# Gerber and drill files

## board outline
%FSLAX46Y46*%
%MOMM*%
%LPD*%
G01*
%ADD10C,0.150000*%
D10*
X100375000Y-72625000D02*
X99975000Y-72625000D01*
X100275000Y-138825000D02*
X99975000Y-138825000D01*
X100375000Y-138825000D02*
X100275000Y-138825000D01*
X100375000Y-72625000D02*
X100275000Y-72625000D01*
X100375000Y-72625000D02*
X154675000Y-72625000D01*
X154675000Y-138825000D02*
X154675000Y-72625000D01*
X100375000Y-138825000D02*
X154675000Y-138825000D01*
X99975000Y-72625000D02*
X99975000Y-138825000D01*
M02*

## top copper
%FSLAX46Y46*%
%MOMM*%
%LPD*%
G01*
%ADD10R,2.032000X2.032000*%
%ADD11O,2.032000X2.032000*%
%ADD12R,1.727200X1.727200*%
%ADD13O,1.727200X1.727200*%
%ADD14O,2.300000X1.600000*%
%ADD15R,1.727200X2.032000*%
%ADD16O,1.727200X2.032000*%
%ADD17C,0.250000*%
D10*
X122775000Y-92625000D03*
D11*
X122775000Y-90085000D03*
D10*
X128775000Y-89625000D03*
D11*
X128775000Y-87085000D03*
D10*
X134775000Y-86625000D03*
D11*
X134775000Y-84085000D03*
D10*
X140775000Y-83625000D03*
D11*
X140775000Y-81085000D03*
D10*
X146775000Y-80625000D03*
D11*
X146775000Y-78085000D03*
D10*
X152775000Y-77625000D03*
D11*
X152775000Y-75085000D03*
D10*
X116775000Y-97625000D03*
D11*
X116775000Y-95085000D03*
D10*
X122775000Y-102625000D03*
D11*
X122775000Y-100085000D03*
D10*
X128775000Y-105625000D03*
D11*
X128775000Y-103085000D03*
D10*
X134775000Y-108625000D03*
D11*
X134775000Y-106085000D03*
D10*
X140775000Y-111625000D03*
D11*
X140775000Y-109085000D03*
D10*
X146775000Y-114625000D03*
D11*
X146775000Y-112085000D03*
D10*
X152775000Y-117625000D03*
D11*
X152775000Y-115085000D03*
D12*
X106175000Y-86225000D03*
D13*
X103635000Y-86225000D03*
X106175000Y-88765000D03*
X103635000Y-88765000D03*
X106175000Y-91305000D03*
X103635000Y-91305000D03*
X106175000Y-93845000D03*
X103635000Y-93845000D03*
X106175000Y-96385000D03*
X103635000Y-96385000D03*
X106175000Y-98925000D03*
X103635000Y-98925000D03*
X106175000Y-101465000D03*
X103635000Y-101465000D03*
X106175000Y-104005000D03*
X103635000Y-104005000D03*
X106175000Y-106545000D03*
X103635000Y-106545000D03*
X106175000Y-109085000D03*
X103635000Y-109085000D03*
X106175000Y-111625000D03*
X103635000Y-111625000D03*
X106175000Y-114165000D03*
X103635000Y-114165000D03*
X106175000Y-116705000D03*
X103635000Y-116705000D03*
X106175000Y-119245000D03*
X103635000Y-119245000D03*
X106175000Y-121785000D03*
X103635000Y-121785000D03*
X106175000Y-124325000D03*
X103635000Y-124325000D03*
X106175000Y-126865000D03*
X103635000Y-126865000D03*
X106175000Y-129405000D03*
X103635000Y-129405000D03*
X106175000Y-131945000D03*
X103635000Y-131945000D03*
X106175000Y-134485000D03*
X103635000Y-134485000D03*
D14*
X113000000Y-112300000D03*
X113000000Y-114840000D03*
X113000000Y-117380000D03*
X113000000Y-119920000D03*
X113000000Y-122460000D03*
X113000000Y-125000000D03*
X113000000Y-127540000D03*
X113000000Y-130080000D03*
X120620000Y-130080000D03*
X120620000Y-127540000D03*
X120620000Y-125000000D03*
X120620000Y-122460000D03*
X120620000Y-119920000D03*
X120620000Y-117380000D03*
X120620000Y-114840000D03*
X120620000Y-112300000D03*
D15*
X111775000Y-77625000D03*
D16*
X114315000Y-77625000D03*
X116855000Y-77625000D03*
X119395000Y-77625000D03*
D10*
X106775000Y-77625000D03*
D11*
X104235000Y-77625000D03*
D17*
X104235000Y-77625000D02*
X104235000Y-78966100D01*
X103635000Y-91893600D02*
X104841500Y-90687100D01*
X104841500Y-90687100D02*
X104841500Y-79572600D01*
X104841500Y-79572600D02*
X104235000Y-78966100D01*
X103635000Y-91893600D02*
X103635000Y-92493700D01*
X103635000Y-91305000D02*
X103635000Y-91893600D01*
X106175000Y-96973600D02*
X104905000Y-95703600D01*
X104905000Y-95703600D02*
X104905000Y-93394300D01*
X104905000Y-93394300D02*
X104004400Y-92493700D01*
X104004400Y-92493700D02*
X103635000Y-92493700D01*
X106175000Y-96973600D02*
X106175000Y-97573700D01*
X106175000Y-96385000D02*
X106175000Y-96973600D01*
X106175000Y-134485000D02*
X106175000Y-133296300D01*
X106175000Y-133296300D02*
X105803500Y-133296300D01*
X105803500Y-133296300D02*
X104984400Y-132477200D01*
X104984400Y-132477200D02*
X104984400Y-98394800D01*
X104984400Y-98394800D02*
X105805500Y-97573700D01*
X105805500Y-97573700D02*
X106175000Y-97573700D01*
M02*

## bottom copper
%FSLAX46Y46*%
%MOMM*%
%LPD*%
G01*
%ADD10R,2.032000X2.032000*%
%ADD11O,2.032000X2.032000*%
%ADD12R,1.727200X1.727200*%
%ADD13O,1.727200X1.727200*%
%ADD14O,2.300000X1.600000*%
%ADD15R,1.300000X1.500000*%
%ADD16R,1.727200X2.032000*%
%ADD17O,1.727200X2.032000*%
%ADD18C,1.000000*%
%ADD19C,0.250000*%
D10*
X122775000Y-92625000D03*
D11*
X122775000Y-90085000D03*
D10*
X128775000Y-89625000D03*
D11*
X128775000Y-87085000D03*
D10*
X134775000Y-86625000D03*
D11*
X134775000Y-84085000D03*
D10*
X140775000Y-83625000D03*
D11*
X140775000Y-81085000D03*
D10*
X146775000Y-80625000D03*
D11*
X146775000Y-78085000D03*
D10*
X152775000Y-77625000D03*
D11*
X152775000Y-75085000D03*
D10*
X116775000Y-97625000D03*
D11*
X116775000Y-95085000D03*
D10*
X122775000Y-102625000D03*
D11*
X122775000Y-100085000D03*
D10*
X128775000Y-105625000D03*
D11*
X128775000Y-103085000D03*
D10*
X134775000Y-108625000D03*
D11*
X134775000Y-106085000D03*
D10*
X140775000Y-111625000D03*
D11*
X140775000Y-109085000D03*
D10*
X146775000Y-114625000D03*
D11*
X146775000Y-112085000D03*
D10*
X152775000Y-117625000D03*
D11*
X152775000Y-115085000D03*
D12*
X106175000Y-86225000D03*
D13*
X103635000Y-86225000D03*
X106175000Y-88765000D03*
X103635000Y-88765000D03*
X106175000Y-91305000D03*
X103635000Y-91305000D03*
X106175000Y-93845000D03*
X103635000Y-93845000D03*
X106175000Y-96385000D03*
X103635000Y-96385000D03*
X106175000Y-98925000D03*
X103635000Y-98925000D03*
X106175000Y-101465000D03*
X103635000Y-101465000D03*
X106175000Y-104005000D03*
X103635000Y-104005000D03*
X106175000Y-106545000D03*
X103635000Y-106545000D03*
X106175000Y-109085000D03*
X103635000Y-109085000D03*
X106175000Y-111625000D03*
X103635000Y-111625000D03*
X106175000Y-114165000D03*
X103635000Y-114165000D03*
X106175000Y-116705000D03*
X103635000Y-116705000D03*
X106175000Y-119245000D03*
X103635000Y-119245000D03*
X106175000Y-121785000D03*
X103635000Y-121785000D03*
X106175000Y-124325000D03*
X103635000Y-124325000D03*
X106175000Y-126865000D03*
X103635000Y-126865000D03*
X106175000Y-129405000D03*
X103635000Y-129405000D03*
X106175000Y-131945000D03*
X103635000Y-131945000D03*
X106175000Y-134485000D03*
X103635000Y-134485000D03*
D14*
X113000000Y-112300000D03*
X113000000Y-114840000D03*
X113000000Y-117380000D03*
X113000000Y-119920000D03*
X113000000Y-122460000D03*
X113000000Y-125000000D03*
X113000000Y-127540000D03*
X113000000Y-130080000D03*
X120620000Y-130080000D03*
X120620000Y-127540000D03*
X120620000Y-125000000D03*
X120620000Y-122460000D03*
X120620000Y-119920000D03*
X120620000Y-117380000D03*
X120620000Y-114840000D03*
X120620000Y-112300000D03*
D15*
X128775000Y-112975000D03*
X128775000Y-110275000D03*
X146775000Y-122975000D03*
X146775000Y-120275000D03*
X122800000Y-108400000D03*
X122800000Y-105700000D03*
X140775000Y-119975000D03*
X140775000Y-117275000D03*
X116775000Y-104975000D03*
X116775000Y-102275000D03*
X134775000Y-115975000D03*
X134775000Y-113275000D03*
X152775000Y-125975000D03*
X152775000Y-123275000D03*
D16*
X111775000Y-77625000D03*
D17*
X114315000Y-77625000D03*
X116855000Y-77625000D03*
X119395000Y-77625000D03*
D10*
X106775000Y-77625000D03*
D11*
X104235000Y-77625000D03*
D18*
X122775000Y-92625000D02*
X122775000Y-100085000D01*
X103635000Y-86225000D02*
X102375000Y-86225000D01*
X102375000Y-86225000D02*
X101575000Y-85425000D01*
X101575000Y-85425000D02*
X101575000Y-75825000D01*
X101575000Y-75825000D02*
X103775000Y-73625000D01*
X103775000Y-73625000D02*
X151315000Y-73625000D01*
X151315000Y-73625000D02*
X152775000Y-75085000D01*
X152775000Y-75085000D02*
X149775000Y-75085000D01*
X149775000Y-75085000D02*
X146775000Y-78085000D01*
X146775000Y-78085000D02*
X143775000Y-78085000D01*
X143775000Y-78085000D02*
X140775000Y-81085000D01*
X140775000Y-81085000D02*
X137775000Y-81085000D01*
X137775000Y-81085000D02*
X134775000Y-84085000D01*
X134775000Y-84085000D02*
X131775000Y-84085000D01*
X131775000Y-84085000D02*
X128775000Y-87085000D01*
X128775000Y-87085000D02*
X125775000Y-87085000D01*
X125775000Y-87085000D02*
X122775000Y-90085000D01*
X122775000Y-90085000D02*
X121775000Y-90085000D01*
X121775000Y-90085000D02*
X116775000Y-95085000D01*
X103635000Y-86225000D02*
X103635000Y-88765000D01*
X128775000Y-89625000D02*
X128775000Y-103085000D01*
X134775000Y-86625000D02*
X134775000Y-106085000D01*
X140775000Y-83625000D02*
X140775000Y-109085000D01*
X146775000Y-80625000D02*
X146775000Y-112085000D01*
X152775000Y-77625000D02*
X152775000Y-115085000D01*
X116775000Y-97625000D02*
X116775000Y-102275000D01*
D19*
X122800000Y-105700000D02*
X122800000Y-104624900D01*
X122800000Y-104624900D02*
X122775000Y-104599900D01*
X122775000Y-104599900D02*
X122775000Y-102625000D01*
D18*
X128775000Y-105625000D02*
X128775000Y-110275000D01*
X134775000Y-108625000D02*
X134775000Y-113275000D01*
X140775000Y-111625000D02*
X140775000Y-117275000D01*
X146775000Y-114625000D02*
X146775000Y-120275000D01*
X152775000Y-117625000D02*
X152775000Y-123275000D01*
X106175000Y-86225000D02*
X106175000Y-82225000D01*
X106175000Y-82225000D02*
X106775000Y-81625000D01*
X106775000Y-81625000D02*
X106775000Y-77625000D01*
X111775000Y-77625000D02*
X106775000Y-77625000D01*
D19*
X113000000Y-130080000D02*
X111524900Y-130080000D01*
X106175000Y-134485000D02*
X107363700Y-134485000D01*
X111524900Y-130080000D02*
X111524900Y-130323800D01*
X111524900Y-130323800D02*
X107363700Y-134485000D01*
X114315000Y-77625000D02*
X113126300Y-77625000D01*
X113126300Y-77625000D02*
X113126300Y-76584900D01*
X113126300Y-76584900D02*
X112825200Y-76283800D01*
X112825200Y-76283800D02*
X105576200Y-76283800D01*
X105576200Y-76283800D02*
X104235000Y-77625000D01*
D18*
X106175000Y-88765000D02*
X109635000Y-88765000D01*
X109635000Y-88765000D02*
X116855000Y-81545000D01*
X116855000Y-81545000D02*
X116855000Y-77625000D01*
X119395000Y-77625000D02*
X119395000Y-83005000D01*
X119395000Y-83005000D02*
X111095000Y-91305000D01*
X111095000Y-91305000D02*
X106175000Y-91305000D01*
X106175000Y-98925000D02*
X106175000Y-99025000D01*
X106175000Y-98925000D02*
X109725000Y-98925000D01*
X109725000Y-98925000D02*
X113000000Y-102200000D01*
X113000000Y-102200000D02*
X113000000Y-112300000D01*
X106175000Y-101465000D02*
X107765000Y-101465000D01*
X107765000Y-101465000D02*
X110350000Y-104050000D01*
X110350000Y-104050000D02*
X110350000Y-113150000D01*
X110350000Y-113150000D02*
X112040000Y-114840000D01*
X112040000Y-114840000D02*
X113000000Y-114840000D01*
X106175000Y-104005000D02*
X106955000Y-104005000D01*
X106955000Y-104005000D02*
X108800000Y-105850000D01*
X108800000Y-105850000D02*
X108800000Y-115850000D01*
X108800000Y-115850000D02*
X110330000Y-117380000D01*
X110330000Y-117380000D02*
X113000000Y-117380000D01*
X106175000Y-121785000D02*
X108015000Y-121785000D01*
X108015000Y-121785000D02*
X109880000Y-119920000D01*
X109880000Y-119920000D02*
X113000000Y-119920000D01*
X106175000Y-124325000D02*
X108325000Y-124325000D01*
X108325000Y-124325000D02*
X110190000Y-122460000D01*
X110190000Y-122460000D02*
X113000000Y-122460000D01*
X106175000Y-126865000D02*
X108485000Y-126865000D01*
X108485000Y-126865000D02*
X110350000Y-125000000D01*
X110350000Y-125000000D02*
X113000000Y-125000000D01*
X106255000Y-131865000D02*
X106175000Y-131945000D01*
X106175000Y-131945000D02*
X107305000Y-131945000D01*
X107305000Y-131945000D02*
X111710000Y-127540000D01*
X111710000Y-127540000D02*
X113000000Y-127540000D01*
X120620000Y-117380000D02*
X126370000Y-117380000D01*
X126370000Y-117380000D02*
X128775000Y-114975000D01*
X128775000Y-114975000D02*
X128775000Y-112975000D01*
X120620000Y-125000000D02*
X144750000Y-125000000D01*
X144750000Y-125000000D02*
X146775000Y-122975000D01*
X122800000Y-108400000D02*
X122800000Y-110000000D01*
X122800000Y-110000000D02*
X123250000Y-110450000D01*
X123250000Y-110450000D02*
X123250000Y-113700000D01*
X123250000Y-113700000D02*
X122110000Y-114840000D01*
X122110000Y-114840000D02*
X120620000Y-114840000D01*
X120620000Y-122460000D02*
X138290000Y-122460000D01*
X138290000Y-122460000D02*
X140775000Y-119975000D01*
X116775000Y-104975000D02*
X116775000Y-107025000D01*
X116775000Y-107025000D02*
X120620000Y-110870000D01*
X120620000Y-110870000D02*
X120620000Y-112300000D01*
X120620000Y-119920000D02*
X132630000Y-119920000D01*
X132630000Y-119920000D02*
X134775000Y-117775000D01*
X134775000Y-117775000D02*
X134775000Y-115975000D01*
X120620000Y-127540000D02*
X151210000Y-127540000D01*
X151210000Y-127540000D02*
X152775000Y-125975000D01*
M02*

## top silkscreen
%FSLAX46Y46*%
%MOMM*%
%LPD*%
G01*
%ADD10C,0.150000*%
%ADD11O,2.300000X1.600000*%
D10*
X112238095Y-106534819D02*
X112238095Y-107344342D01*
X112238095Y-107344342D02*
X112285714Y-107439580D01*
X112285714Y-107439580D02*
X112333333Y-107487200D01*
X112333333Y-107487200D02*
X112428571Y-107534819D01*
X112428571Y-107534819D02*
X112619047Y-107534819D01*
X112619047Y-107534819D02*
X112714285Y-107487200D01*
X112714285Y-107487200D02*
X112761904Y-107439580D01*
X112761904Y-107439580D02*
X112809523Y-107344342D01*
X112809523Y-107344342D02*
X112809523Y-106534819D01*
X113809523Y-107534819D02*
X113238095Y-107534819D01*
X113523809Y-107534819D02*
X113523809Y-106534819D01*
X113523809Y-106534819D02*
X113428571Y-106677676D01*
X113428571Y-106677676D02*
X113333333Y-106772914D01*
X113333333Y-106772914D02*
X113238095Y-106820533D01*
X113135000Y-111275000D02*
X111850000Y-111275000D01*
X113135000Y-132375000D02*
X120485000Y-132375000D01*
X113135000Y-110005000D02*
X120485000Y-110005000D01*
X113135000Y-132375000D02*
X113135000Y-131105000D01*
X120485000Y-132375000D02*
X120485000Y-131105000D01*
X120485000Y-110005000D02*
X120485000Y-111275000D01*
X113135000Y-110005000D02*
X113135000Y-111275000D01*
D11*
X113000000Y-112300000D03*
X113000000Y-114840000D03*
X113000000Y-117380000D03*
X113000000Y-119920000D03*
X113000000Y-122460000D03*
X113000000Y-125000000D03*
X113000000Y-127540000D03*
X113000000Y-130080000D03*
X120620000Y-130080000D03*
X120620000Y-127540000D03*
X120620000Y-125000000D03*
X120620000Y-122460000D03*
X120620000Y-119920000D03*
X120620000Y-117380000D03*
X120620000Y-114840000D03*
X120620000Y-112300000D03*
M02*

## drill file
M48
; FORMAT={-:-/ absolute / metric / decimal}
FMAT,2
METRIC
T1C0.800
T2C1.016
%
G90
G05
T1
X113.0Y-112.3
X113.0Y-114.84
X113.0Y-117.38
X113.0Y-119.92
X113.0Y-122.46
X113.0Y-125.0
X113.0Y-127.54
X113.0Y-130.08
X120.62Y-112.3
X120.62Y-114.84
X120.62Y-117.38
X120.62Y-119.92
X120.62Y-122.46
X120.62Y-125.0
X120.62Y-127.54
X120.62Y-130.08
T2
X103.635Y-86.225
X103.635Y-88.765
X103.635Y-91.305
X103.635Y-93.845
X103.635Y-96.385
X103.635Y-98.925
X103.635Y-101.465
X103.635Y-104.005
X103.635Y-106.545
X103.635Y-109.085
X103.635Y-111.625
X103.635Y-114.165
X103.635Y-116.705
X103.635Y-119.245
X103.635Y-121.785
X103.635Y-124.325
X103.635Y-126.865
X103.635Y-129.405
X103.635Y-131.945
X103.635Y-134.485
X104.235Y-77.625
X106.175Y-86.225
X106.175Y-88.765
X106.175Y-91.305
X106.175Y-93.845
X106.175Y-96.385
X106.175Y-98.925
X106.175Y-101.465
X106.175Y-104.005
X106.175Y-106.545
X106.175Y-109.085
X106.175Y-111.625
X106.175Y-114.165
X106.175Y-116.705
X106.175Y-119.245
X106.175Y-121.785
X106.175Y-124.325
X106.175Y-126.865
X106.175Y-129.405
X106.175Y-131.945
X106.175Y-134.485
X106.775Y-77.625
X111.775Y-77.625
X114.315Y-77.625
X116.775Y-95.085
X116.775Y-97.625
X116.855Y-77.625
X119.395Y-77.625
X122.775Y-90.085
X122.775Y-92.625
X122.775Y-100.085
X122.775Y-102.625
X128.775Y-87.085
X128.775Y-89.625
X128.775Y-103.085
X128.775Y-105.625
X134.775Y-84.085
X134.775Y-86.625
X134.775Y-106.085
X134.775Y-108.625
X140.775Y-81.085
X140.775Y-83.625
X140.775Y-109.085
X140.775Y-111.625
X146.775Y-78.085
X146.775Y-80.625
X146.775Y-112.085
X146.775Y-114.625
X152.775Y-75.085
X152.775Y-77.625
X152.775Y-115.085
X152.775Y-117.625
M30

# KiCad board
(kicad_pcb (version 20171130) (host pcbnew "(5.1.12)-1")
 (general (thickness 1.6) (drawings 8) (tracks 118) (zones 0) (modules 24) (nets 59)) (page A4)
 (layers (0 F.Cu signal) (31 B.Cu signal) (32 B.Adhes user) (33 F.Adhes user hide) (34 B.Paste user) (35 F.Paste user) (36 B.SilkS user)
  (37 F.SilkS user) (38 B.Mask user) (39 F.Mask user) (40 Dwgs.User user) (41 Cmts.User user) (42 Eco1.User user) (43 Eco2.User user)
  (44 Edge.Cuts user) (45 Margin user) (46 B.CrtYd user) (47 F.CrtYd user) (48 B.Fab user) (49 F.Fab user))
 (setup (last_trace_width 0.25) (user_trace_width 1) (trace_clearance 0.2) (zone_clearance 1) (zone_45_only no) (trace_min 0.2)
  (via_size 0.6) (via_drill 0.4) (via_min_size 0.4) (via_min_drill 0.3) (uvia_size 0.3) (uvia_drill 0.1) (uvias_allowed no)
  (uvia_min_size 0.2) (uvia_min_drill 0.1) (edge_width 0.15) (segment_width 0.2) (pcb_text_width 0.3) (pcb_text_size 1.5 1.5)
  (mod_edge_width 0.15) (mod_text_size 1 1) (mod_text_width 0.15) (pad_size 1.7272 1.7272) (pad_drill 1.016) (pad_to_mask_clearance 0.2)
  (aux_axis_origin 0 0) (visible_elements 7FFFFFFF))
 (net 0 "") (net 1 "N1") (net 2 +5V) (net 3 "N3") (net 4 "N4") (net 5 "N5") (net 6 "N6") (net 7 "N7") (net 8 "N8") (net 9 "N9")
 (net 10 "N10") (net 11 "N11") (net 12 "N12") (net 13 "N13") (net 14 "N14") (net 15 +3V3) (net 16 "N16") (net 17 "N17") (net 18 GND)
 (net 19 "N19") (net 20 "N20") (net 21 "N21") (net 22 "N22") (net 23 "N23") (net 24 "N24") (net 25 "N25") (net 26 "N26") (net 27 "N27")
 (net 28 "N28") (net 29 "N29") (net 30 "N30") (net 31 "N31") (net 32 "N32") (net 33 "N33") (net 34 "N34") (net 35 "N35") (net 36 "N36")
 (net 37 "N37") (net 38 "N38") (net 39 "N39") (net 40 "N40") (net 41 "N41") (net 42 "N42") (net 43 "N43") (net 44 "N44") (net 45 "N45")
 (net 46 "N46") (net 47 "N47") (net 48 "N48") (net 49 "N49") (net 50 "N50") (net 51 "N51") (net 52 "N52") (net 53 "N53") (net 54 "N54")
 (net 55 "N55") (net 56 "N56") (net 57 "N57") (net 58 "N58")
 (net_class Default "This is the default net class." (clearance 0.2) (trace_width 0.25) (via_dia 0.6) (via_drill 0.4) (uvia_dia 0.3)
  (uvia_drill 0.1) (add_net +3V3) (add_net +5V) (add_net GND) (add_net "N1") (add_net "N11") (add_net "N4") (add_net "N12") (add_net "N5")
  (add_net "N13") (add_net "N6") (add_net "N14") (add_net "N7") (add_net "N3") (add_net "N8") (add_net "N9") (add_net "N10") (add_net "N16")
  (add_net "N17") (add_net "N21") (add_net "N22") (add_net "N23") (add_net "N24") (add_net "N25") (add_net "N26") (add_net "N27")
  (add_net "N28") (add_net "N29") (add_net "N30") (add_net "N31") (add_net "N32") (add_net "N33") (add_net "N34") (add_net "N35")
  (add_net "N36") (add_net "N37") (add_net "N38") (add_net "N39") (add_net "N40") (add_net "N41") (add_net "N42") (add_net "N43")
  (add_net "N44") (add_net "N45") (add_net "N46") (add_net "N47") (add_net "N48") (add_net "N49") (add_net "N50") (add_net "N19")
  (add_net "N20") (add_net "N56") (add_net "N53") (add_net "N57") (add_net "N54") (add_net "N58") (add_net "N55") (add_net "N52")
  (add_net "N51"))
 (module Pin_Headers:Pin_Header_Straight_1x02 (layer B.Cu) (at 122.775 92.625)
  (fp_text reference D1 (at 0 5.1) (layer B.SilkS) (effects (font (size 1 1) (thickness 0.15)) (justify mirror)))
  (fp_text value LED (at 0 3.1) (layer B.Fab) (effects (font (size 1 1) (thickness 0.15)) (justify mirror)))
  (pad 1 thru_hole rect (at 0 0) (size 2.032 2.032) (drill 1.016) (layers *.Cu *.Mask B.SilkS) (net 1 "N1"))
  (pad 2 thru_hole oval (at 0 -2.54) (size 2.032 2.032) (drill 1.016) (layers *.Cu *.Mask B.SilkS) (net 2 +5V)))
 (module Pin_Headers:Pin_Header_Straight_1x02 (layer B.Cu) (at 128.775 89.625)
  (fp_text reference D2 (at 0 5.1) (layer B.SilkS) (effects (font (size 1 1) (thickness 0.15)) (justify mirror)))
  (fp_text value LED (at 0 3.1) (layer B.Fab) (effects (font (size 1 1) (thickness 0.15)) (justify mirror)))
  (pad 1 thru_hole rect (at 0 0) (size 2.032 2.032) (drill 1.016) (layers *.Cu *.Mask B.SilkS) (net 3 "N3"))
  (pad 2 thru_hole oval (at 0 -2.54) (size 2.032 2.032) (drill 1.016) (layers *.Cu *.Mask B.SilkS) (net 2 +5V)))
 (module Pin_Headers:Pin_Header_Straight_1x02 (layer B.Cu) (at 134.775 86.625)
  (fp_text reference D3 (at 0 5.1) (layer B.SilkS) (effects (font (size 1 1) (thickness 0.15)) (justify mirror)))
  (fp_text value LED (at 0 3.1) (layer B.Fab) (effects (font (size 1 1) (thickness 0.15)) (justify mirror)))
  (pad 1 thru_hole rect (at 0 0) (size 2.032 2.032) (drill 1.016) (layers *.Cu *.Mask B.SilkS) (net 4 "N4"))
  (pad 2 thru_hole oval (at 0 -2.54) (size 2.032 2.032) (drill 1.016) (layers *.Cu *.Mask B.SilkS) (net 2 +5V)))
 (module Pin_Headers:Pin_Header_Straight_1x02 (layer B.Cu) (at 140.775 83.625)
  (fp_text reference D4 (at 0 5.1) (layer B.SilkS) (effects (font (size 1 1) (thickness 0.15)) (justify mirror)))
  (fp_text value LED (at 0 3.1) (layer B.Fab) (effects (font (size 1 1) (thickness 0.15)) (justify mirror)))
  (pad 1 thru_hole rect (at 0 0) (size 2.032 2.032) (drill 1.016) (layers *.Cu *.Mask B.SilkS) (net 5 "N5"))
  (pad 2 thru_hole oval (at 0 -2.54) (size 2.032 2.032) (drill 1.016) (layers *.Cu *.Mask B.SilkS) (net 2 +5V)))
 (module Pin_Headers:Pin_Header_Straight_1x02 (layer B.Cu) (at 146.775 80.625)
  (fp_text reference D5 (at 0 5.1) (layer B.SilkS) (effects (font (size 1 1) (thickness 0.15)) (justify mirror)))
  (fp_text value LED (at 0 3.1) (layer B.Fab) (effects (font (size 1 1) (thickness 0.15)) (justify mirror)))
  (pad 1 thru_hole rect (at 0 0) (size 2.032 2.032) (drill 1.016) (layers *.Cu *.Mask B.SilkS) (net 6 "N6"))
  (pad 2 thru_hole oval (at 0 -2.54) (size 2.032 2.032) (drill 1.016) (layers *.Cu *.Mask B.SilkS) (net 2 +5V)))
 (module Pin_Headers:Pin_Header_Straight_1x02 (layer B.Cu) (at 152.775 77.625)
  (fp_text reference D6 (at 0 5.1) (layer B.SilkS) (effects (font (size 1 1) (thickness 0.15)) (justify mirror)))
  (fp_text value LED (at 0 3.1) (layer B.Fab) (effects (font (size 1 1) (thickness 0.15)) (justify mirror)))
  (pad 1 thru_hole rect (at 0 0) (size 2.032 2.032) (drill 1.016) (layers *.Cu *.Mask B.SilkS) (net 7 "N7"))
  (pad 2 thru_hole oval (at 0 -2.54) (size 2.032 2.032) (drill 1.016) (layers *.Cu *.Mask B.SilkS) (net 2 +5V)))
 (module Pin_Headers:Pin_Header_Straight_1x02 (layer B.Cu) (at 116.775 97.625)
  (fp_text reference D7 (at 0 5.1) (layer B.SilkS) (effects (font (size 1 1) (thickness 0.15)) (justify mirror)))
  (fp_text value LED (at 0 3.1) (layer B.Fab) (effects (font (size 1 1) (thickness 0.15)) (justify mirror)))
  (pad 1 thru_hole rect (at 0 0) (size 2.032 2.032) (drill 1.016) (layers *.Cu *.Mask B.SilkS) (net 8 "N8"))
  (pad 2 thru_hole oval (at 0 -2.54) (size 2.032 2.032) (drill 1.016) (layers *.Cu *.Mask B.SilkS) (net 2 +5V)))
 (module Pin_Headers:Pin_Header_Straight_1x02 (layer B.Cu) (at 122.775 102.625)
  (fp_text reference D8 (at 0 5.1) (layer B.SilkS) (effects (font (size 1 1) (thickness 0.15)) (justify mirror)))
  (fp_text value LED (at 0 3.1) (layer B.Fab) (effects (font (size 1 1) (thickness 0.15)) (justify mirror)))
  (pad 1 thru_hole rect (at 0 0) (size 2.032 2.032) (drill 1.016) (layers *.Cu *.Mask B.SilkS) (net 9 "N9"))
  (pad 2 thru_hole oval (at 0 -2.54) (size 2.032 2.032) (drill 1.016) (layers *.Cu *.Mask B.SilkS) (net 1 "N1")))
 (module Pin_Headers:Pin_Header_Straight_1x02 (layer B.Cu) (at 128.775 105.625)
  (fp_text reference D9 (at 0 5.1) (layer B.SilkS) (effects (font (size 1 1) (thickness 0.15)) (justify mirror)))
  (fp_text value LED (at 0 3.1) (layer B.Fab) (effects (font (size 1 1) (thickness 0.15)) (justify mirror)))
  (pad 1 thru_hole rect (at 0 0) (size 2.032 2.032) (drill 1.016) (layers *.Cu *.Mask B.SilkS) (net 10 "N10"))
  (pad 2 thru_hole oval (at 0 -2.54) (size 2.032 2.032) (drill 1.016) (layers *.Cu *.Mask B.SilkS) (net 3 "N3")))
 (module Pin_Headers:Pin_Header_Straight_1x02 (layer B.Cu) (at 134.775 108.625)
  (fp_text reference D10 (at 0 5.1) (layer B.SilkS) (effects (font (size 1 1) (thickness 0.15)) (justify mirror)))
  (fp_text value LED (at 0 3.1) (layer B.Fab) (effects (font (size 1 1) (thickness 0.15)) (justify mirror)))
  (pad 1 thru_hole rect (at 0 0) (size 2.032 2.032) (drill 1.016) (layers *.Cu *.Mask B.SilkS) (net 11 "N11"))
  (pad 2 thru_hole oval (at 0 -2.54) (size 2.032 2.032) (drill 1.016) (layers *.Cu *.Mask B.SilkS) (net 4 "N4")))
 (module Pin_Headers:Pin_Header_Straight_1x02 (layer B.Cu) (at 140.775 111.625)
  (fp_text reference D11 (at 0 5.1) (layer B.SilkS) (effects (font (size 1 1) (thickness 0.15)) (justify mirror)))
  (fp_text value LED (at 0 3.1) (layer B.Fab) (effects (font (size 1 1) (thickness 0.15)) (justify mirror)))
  (pad 1 thru_hole rect (at 0 0) (size 2.032 2.032) (drill 1.016) (layers *.Cu *.Mask B.SilkS) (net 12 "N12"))
  (pad 2 thru_hole oval (at 0 -2.54) (size 2.032 2.032) (drill 1.016) (layers *.Cu *.Mask B.SilkS) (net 5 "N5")))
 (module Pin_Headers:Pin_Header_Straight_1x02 (layer B.Cu) (at 146.775 114.625)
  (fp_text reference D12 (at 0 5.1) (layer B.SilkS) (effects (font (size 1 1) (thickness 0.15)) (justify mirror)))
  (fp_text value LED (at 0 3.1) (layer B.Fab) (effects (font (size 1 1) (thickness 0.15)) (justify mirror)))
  (pad 1 thru_hole rect (at 0 0) (size 2.032 2.032) (drill 1.016) (layers *.Cu *.Mask B.SilkS) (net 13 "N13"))
  (pad 2 thru_hole oval (at 0 -2.54) (size 2.032 2.032) (drill 1.016) (layers *.Cu *.Mask B.SilkS) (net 6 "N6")))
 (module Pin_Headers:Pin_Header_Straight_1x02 (layer B.Cu) (at 152.775 117.625)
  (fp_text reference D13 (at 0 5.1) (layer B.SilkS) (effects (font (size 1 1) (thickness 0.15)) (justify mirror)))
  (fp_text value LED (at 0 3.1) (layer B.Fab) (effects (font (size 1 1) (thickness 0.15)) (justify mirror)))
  (pad 1 thru_hole rect (at 0 0) (size 2.032 2.032) (drill 1.016) (layers *.Cu *.Mask B.SilkS) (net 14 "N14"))
  (pad 2 thru_hole oval (at 0 -2.54) (size 2.032 2.032) (drill 1.016) (layers *.Cu *.Mask B.SilkS) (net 7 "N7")))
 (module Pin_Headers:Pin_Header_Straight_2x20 (layer B.Cu) (at 106.175 86.225 180)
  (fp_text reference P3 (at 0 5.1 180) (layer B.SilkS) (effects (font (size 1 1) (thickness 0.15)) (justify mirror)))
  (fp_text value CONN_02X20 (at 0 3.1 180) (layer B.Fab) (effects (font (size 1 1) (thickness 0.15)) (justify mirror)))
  (pad 1 thru_hole rect (at 0 0 180) (size 1.7272 1.7272) (drill 1.016) (layers *.Cu *.Mask B.SilkS) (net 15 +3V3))
  (pad 2 thru_hole oval (at 2.54 0 180) (size 1.7272 1.7272) (drill 1.016) (layers *.Cu *.Mask B.SilkS) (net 2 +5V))
  (pad 3 thru_hole oval (at 0 -2.54 180) (size 1.7272 1.7272) (drill 1.016) (layers *.Cu *.Mask B.SilkS) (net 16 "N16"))
  (pad 4 thru_hole oval (at 2.54 -2.54 180) (size 1.7272 1.7272) (drill 1.016) (layers *.Cu *.Mask B.SilkS) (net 2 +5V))
  (pad 5 thru_hole oval (at 0 -5.08 180) (size 1.7272 1.7272) (drill 1.016) (layers *.Cu *.Mask B.SilkS) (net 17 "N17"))
  (pad 6 thru_hole oval (at 2.54 -5.08 180) (size 1.7272 1.7272) (drill 1.016) (layers *.Cu *.Mask B.SilkS) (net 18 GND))
  (pad 7 thru_hole oval (at 0 -7.62 180) (size 1.7272 1.7272) (drill 1.016) (layers *.Cu *.Mask B.SilkS) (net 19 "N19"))
  (pad 8 thru_hole oval (at 2.54 -7.62 180) (size 1.7272 1.7272) (drill 1.016) (layers *.Cu *.Mask B.SilkS) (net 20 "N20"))
  (pad 9 thru_hole oval (at 0 -10.16 180) (size 1.7272 1.7272) (drill 1.016) (layers *.Cu *.Mask B.SilkS) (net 18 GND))
  (pad 10 thru_hole oval (at 2.54 -10.16 180) (size 1.7272 1.7272) (drill 1.016) (layers *.Cu *.Mask B.SilkS) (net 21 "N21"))
  (pad 11 thru_hole oval (at 0 -12.7 180) (size 1.7272 1.7272) (drill 1.016) (layers *.Cu *.Mask B.SilkS) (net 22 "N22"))
  (pad 12 thru_hole oval (at 2.54 -12.7 180) (size 1.7272 1.7272) (drill 1.016) (layers *.Cu *.Mask B.SilkS) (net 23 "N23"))
  (pad 13 thru_hole oval (at 0 -15.24 180) (size 1.7272 1.7272) (drill 1.016) (layers *.Cu *.Mask B.SilkS) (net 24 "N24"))
  (pad 14 thru_hole oval (at 2.54 -15.24 180) (size 1.7272 1.7272) (drill 1.016) (layers *.Cu *.Mask B.SilkS) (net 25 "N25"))
  (pad 15 thru_hole oval (at 0 -17.78 180) (size 1.7272 1.7272) (drill 1.016) (layers *.Cu *.Mask B.SilkS) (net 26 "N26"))
  (pad 16 thru_hole oval (at 2.54 -17.78 180) (size 1.7272 1.7272) (drill 1.016) (layers *.Cu *.Mask B.SilkS) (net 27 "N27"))
  (pad 17 thru_hole oval (at 0 -20.32 180) (size 1.7272 1.7272) (drill 1.016) (layers *.Cu *.Mask B.SilkS) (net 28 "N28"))
  (pad 18 thru_hole oval (at 2.54 -20.32 180) (size 1.7272 1.7272) (drill 1.016) (layers *.Cu *.Mask B.SilkS) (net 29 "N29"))
  (pad 19 thru_hole oval (at 0 -22.86 180) (size 1.7272 1.7272) (drill 1.016) (layers *.Cu *.Mask B.SilkS) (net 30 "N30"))
  (pad 20 thru_hole oval (at 2.54 -22.86 180) (size 1.7272 1.7272) (drill 1.016) (layers *.Cu *.Mask B.SilkS) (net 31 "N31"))
  (pad 21 thru_hole oval (at 0 -25.4 180) (size 1.7272 1.7272) (drill 1.016) (layers *.Cu *.Mask B.SilkS) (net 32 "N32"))
  (pad 22 thru_hole oval (at 2.54 -25.4 180) (size 1.7272 1.7272) (drill 1.016) (layers *.Cu *.Mask B.SilkS) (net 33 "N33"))
  (pad 23 thru_hole oval (at 0 -27.94 180) (size 1.7272 1.7272) (drill 1.016) (layers *.Cu *.Mask B.SilkS) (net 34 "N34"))
  (pad 24 thru_hole oval (at 2.54 -27.94 180) (size 1.7272 1.7272) (drill 1.016) (layers *.Cu *.Mask B.SilkS) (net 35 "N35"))
  (pad 25 thru_hole oval (at 0 -30.48 180) (size 1.7272 1.7272) (drill 1.016) (layers *.Cu *.Mask B.SilkS) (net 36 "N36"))
  (pad 26 thru_hole oval (at 2.54 -30.48 180) (size 1.7272 1.7272) (drill 1.016) (layers *.Cu *.Mask B.SilkS) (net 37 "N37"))
  (pad 27 thru_hole oval (at 0 -33.02 180) (size 1.7272 1.7272) (drill 1.016) (layers *.Cu *.Mask B.SilkS) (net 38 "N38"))
  (pad 28 thru_hole oval (at 2.54 -33.02 180) (size 1.7272 1.7272) (drill 1.016) (layers *.Cu *.Mask B.SilkS) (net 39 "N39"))
  (pad 29 thru_hole oval (at 0 -35.56 180) (size 1.7272 1.7272) (drill 1.016) (layers *.Cu *.Mask B.SilkS) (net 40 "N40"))
  (pad 30 thru_hole oval (at 2.54 -35.56 180) (size 1.7272 1.7272) (drill 1.016) (layers *.Cu *.Mask B.SilkS) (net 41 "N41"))
  (pad 31 thru_hole oval (at 0 -38.1 180) (size 1.7272 1.7272) (drill 1.016) (layers *.Cu *.Mask B.SilkS) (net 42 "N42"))
  (pad 32 thru_hole oval (at 2.54 -38.1 180) (size 1.7272 1.7272) (drill 1.016) (layers *.Cu *.Mask B.SilkS) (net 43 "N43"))
  (pad 33 thru_hole oval (at 0 -40.64 180) (size 1.7272 1.7272) (drill 1.016) (layers *.Cu *.Mask B.SilkS) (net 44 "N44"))
  (pad 34 thru_hole oval (at 2.54 -40.64 180) (size 1.7272 1.7272) (drill 1.016) (layers *.Cu *.Mask B.SilkS) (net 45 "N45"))
  (pad 35 thru_hole oval (at 0 -43.18 180) (size 1.7272 1.7272) (drill 1.016) (layers *.Cu *.Mask B.SilkS) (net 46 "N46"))
  (pad 36 thru_hole oval (at 2.54 -43.18 180) (size 1.7272 1.7272) (drill 1.016) (layers *.Cu *.Mask B.SilkS) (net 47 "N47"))
  (pad 37 thru_hole oval (at 0 -45.72 180) (size 1.7272 1.7272) (drill 1.016) (layers *.Cu *.Mask B.SilkS) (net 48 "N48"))
  (pad 38 thru_hole oval (at 2.54 -45.72 180) (size 1.7272 1.7272) (drill 1.016) (layers *.Cu *.Mask B.SilkS) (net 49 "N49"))
  (pad 39 thru_hole oval (at 0 -48.26 180) (size 1.7272 1.7272) (drill 1.016) (layers *.Cu *.Mask B.SilkS) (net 18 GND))
  (pad 40 thru_hole oval (at 2.54 -48.26 180) (size 1.7272 1.7272) (drill 1.016) (layers *.Cu *.Mask B.SilkS) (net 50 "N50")))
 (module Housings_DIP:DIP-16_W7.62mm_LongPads (layer F.Cu) (at 113 112.3)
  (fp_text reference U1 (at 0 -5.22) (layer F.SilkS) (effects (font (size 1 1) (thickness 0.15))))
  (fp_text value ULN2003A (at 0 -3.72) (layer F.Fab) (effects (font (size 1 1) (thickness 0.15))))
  (fp_line (start 0.135 -1.025) (end -1.15 -1.025) (layer F.SilkS) (width 0.15))
  (fp_line (start 0.135 20.075) (end 7.485 20.075) (layer F.SilkS) (width 0.15))
  (fp_line (start 0.135 -2.295) (end 7.485 -2.295) (layer F.SilkS) (width 0.15))
  (fp_line (start 0.135 20.075) (end 0.135 18.805) (layer F.SilkS) (width 0.15))
  (fp_line (start 7.485 20.075) (end 7.485 18.805) (layer F.SilkS) (width 0.15))
  (fp_line (start 7.485 -2.295) (end 7.485 -1.025) (layer F.SilkS) (width 0.15))
  (fp_line (start 0.135 -2.295) (end 0.135 -1.025) (layer F.SilkS) (width 0.15))
  (pad 1 thru_hole oval (at 0 0) (size 2.3 1.6) (drill 0.8) (layers *.Cu *.Mask F.SilkS) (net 22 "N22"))
  (pad 2 thru_hole oval (at 0 2.54) (size 2.3 1.6) (drill 0.8) (layers *.Cu *.Mask F.SilkS) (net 24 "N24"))
  (pad 3 thru_hole oval (at 0 5.08) (size 2.3 1.6) (drill 0.8) (layers *.Cu *.Mask F.SilkS) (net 26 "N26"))
  (pad 4 thru_hole oval (at 0 7.62) (size 2.3 1.6) (drill 0.8) (layers *.Cu *.Mask F.SilkS) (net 40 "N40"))
  (pad 5 thru_hole oval (at 0 10.16) (size 2.3 1.6) (drill 0.8) (layers *.Cu *.Mask F.SilkS) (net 42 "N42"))
  (pad 6 thru_hole oval (at 0 12.7) (size 2.3 1.6) (drill 0.8) (layers *.Cu *.Mask F.SilkS) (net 44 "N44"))
  (pad 7 thru_hole oval (at 0 15.24) (size 2.3 1.6) (drill 0.8) (layers *.Cu *.Mask F.SilkS) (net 48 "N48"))
  (pad 8 thru_hole oval (at 0 17.78) (size 2.3 1.6) (drill 0.8) (layers *.Cu *.Mask F.SilkS) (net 18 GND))
  (pad 9 thru_hole oval (at 7.62 17.78) (size 2.3 1.6) (drill 0.8) (layers *.Cu *.Mask F.SilkS) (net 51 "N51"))
  (pad 10 thru_hole oval (at 7.62 15.24) (size 2.3 1.6) (drill 0.8) (layers *.Cu *.Mask F.SilkS) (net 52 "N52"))
  (pad 11 thru_hole oval (at 7.62 12.7) (size 2.3 1.6) (drill 0.8) (layers *.Cu *.Mask F.SilkS) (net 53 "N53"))
  (pad 12 thru_hole oval (at 7.62 10.16) (size 2.3 1.6) (drill 0.8) (layers *.Cu *.Mask F.SilkS) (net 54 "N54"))
  (pad 13 thru_hole oval (at 7.62 7.62) (size 2.3 1.6) (drill 0.8) (layers *.Cu *.Mask F.SilkS) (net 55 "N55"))
  (pad 14 thru_hole oval (at 7.62 5.08) (size 2.3 1.6) (drill 0.8) (layers *.Cu *.Mask F.SilkS) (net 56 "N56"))
  (pad 15 thru_hole oval (at 7.62 2.54) (size 2.3 1.6) (drill 0.8) (layers *.Cu *.Mask F.SilkS) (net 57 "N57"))
  (pad 16 thru_hole oval (at 7.62 0) (size 2.3 1.6) (drill 0.8) (layers *.Cu *.Mask F.SilkS) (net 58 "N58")))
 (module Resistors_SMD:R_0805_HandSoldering (layer B.Cu) (at 128.775 111.625 90)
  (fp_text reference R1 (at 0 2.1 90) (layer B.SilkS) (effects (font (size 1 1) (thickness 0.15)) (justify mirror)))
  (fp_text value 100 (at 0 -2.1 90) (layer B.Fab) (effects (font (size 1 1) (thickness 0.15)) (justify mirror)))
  (pad 1 smd rect (at -1.35 0 90) (size 1.5 1.3) (layers B.Cu B.Paste B.Mask) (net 56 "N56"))
  (pad 2 smd rect (at 1.35 0 90) (size 1.5 1.3) (layers B.Cu B.Paste B.Mask) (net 10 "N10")))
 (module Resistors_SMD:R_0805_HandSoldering (layer B.Cu) (at 146.775 121.625 90)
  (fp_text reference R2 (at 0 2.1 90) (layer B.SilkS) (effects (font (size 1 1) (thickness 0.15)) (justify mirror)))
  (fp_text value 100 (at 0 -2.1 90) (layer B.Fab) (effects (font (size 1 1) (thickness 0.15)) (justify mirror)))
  (pad 1 smd rect (at -1.35 0 90) (size 1.5 1.3) (layers B.Cu B.Paste B.Mask) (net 53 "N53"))
  (pad 2 smd rect (at 1.35 0 90) (size 1.5 1.3) (layers B.Cu B.Paste B.Mask) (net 13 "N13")))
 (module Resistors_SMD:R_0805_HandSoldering (layer B.Cu) (at 122.8 107.05 90)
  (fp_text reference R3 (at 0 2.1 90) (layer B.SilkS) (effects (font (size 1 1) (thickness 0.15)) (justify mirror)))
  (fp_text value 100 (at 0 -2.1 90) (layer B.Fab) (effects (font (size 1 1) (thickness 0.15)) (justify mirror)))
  (pad 1 smd rect (at -1.35 0 90) (size 1.5 1.3) (layers B.Cu B.Paste B.Mask) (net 57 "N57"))
  (pad 2 smd rect (at 1.35 0 90) (size 1.5 1.3) (layers B.Cu B.Paste B.Mask) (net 9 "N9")))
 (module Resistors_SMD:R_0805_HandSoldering (layer B.Cu) (at 140.775 118.625 90)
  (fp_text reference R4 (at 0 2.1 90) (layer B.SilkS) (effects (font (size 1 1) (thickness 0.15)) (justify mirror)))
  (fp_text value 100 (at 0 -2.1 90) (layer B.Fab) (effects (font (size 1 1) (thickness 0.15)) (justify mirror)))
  (pad 1 smd rect (at -1.35 0 90) (size 1.5 1.3) (layers B.Cu B.Paste B.Mask) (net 54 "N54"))
  (pad 2 smd rect (at 1.35 0 90) (size 1.5 1.3) (layers B.Cu B.Paste B.Mask) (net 12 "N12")))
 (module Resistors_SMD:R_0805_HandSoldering (layer B.Cu) (at 116.775 103.625 90)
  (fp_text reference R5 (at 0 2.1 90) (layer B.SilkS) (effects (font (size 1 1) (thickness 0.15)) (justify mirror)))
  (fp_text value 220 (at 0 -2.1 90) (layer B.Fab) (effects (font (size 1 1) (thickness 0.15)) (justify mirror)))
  (pad 1 smd rect (at -1.35 0 90) (size 1.5 1.3) (layers B.Cu B.Paste B.Mask) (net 58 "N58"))
  (pad 2 smd rect (at 1.35 0 90) (size 1.5 1.3) (layers B.Cu B.Paste B.Mask) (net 8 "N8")))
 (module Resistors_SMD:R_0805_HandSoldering (layer B.Cu) (at 134.775 114.625 90)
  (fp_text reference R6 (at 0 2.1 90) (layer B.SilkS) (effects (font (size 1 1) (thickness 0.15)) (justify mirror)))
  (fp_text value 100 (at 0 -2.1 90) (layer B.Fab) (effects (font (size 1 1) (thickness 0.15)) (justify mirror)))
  (pad 1 smd rect (at -1.35 0 90) (size 1.5 1.3) (layers B.Cu B.Paste B.Mask) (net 55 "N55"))
  (pad 2 smd rect (at 1.35 0 90) (size 1.5 1.3) (layers B.Cu B.Paste B.Mask) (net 11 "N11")))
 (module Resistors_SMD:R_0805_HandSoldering (layer B.Cu) (at 152.775 124.625 90)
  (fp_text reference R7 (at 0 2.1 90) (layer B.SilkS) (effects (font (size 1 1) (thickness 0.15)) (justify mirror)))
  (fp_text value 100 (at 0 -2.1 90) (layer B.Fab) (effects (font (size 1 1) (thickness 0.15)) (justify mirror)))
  (pad 1 smd rect (at -1.35 0 90) (size 1.5 1.3) (layers B.Cu B.Paste B.Mask) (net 52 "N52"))
  (pad 2 smd rect (at 1.35 0 90) (size 1.5 1.3) (layers B.Cu B.Paste B.Mask) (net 14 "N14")))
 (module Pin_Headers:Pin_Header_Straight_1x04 (layer B.Cu) (at 111.775 77.625 270)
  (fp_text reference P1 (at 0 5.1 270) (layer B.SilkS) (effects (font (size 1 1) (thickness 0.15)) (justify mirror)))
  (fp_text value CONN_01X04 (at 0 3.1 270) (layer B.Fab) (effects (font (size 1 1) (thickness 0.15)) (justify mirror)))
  (pad 1 thru_hole rect (at 0 0 270) (size 2.032 1.7272) (drill 1.016) (layers *.Cu *.Mask B.SilkS) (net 15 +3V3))
  (pad 2 thru_hole oval (at 0 -2.54 270) (size 2.032 1.7272) (drill 1.016) (layers *.Cu *.Mask B.SilkS) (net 18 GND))
  (pad 3 thru_hole oval (at 0 -5.08 270) (size 2.032 1.7272) (drill 1.016) (layers *.Cu *.Mask B.SilkS) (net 16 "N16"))
  (pad 4 thru_hole oval (at 0 -7.62 270) (size 2.032 1.7272) (drill 1.016) (layers *.Cu *.Mask B.SilkS) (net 17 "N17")))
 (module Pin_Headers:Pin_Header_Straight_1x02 (layer B.Cu) (at 106.775 77.625 90)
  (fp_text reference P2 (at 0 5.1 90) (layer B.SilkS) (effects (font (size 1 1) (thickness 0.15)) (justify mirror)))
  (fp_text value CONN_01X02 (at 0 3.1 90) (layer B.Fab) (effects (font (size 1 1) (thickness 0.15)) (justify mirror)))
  (pad 1 thru_hole rect (at 0 0 90) (size 2.032 2.032) (drill 1.016) (layers *.Cu *.Mask B.SilkS) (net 15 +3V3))
  (pad 2 thru_hole oval (at 0 -2.54 90) (size 2.032 2.032) (drill 1.016) (layers *.Cu *.Mask B.SilkS) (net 18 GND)))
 (gr_line (start 100.375 72.625) (end 99.975 72.625) (angle 90) (layer Edge.Cuts) (width 0.15))
 (gr_line (start 100.275 138.825) (end 99.975 138.825) (angle 90) (layer Edge.Cuts) (width 0.15))
 (gr_line (start 100.375 138.825) (end 100.275 138.825) (angle 90) (layer Edge.Cuts) (width 0.15))
 (gr_line (start 100.375 72.625) (end 100.275 72.625) (angle 90) (layer Edge.Cuts) (width 0.15))
 (gr_line (start 100.375 72.625) (end 154.675 72.625) (angle 90) (layer Edge.Cuts) (width 0.15))
 (gr_line (start 154.675 138.825) (end 154.675 72.625) (angle 90) (layer Edge.Cuts) (width 0.15))
 (gr_line (start 100.375 138.825) (end 154.675 138.825) (angle 90) (layer Edge.Cuts) (width 0.15))
 (gr_line (start 99.975 72.625) (end 99.975 138.825) (angle 90) (layer Edge.Cuts) (width 0.15))
 (segment (start 122.775 92.625) (end 122.775 100.085) (width 1) (layer B.Cu) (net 1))
 (segment (start 103.635 86.225) (end 102.375 86.225) (width 1) (layer B.Cu) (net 2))
 (segment (start 102.375 86.225) (end 101.575 85.425) (width 1) (layer B.Cu) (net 2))
 (segment (start 101.575 85.425) (end 101.575 75.825) (width 1) (layer B.Cu) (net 2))
 (segment (start 101.575 75.825) (end 103.775 73.625) (width 1) (layer B.Cu) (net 2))
 (segment (start 103.775 73.625) (end 151.315 73.625) (width 1) (layer B.Cu) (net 2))
 (segment (start 151.315 73.625) (end 152.775 75.085) (width 1) (layer B.Cu) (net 2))
 (segment (start 152.775 75.085) (end 149.775 75.085) (width 1) (layer B.Cu) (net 2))
 (segment (start 149.775 75.085) (end 146.775 78.085) (width 1) (layer B.Cu) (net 2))
 (segment (start 146.775 78.085) (end 143.775 78.085) (width 1) (layer B.Cu) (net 2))
 (segment (start 143.775 78.085) (end 140.775 81.085) (width 1) (layer B.Cu) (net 2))
 (segment (start 140.775 81.085) (end 137.775 81.085) (width 1) (layer B.Cu) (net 2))
 (segment (start 137.775 81.085) (end 134.775 84.085) (width 1) (layer B.Cu) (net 2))
 (segment (start 134.775 84.085) (end 131.775 84.085) (width 1) (layer B.Cu) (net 2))
 (segment (start 131.775 84.085) (end 128.775 87.085) (width 1) (layer B.Cu) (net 2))
 (segment (start 128.775 87.085) (end 125.775 87.085) (width 1) (layer B.Cu) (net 2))
 (segment (start 125.775 87.085) (end 122.775 90.085) (width 1) (layer B.Cu) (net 2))
 (segment (start 122.775 90.085) (end 121.775 90.085) (width 1) (layer B.Cu) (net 2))
 (segment (start 121.775 90.085) (end 116.775 95.085) (width 1) (layer B.Cu) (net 2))
 (segment (start 103.635 86.225) (end 103.635 88.765) (width 1) (layer B.Cu) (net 2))
 (segment (start 128.775 89.625) (end 128.775 103.085) (width 1) (layer B.Cu) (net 3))
 (segment (start 134.775 86.625) (end 134.775 106.085) (width 1) (layer B.Cu) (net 4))
 (segment (start 140.775 83.625) (end 140.775 109.085) (width 1) (layer B.Cu) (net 5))
 (segment (start 146.775 80.625) (end 146.775 112.085) (width 1) (layer B.Cu) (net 6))
 (segment (start 152.775 77.625) (end 152.775 115.085) (width 1) (layer B.Cu) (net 7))
 (segment (start 116.775 97.625) (end 116.775 102.275) (width 1) (layer B.Cu) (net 8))
 (segment (start 122.8 105.7) (end 122.8 104.6249) (width 0.25) (layer B.Cu) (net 9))
 (segment (start 122.8 104.6249) (end 122.775 104.5999) (width 0.25) (layer B.Cu) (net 9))
 (segment (start 122.775 104.5999) (end 122.775 102.625) (width 0.25) (layer B.Cu) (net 9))
 (segment (start 128.775 105.625) (end 128.775 110.275) (width 1) (layer B.Cu) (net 10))
 (segment (start 134.775 108.625) (end 134.775 113.275) (width 1) (layer B.Cu) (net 11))
 (segment (start 140.775 111.625) (end 140.775 117.275) (width 1) (layer B.Cu) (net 12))
 (segment (start 146.775 114.625) (end 146.775 120.275) (width 1) (layer B.Cu) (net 13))
 (segment (start 152.775 117.625) (end 152.775 123.275) (width 1) (layer B.Cu) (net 14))
 (segment (start 106.175 86.225) (end 106.175 82.225) (width 1) (layer B.Cu) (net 15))
 (segment (start 106.175 82.225) (end 106.775 81.625) (width 1) (layer B.Cu) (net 15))
 (segment (start 106.775 81.625) (end 106.775 77.625) (width 1) (layer B.Cu) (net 15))
 (segment (start 111.775 77.625) (end 106.775 77.625) (width 1) (layer B.Cu) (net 15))
 (segment (start 104.235 77.625) (end 104.235 78.9661) (width 0.25) (layer F.Cu) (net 18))
 (segment (start 103.635 91.8936) (end 104.8415 90.6871) (width 0.25) (layer F.Cu) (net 18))
 (segment (start 104.8415 90.6871) (end 104.8415 79.5726) (width 0.25) (layer F.Cu) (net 18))
 (segment (start 104.8415 79.5726) (end 104.235 78.9661) (width 0.25) (layer F.Cu) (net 18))
 (segment (start 103.635 91.8936) (end 103.635 92.4937) (width 0.25) (layer F.Cu) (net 18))
 (segment (start 103.635 91.305) (end 103.635 91.8936) (width 0.25) (layer F.Cu) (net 18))
 (segment (start 106.175 96.9736) (end 104.905 95.7036) (width 0.25) (layer F.Cu) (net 18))
 (segment (start 104.905 95.7036) (end 104.905 93.3943) (width 0.25) (layer F.Cu) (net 18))
 (segment (start 104.905 93.3943) (end 104.0044 92.4937) (width 0.25) (layer F.Cu) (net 18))
 (segment (start 104.0044 92.4937) (end 103.635 92.4937) (width 0.25) (layer F.Cu) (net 18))
 (segment (start 106.175 96.9736) (end 106.175 97.5737) (width 0.25) (layer F.Cu) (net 18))
 (segment (start 106.175 96.385) (end 106.175 96.9736) (width 0.25) (layer F.Cu) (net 18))
 (segment (start 106.175 134.485) (end 106.175 133.2963) (width 0.25) (layer F.Cu) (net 18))
 (segment (start 106.175 133.2963) (end 105.8035 133.2963) (width 0.25) (layer F.Cu) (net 18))
 (segment (start 105.8035 133.2963) (end 104.9844 132.4772) (width 0.25) (layer F.Cu) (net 18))
 (segment (start 104.9844 132.4772) (end 104.9844 98.3948) (width 0.25) (layer F.Cu) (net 18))
 (segment (start 104.9844 98.3948) (end 105.8055 97.5737) (width 0.25) (layer F.Cu) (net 18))
 (segment (start 105.8055 97.5737) (end 106.175 97.5737) (width 0.25) (layer F.Cu) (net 18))
 (segment (start 113 130.08) (end 111.5249 130.08) (width 0.25) (layer B.Cu) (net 18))
 (segment (start 106.175 134.485) (end 107.3637 134.485) (width 0.25) (layer B.Cu) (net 18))
 (segment (start 111.5249 130.08) (end 111.5249 130.3238) (width 0.25) (layer B.Cu) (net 18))
 (segment (start 111.5249 130.3238) (end 107.3637 134.485) (width 0.25) (layer B.Cu) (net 18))
 (segment (start 114.315 77.625) (end 113.1263 77.625) (width 0.25) (layer B.Cu) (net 18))
 (segment (start 113.1263 77.625) (end 113.1263 76.5849) (width 0.25) (layer B.Cu) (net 18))
 (segment (start 113.1263 76.5849) (end 112.8252 76.2838) (width 0.25) (layer B.Cu) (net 18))
 (segment (start 112.8252 76.2838) (end 105.5762 76.2838) (width 0.25) (layer B.Cu) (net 18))
 (segment (start 105.5762 76.2838) (end 104.235 77.625) (width 0.25) (layer B.Cu) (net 18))
 (segment (start 106.175 88.765) (end 109.635 88.765) (width 1) (layer B.Cu) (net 16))
 (segment (start 109.635 88.765) (end 116.855 81.545) (width 1) (layer B.Cu) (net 16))
 (segment (start 116.855 81.545) (end 116.855 77.625) (width 1) (layer B.Cu) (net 16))
 (segment (start 119.395 77.625) (end 119.395 83.005) (width 1) (layer B.Cu) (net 17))
 (segment (start 119.395 83.005) (end 111.095 91.305) (width 1) (layer B.Cu) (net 17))
 (segment (start 111.095 91.305) (end 106.175 91.305) (width 1) (layer B.Cu) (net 17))
 (segment (start 106.175 98.925) (end 106.175 99.025) (width 1) (layer B.Cu) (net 22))
 (segment (start 106.175 98.925) (end 109.725 98.925) (width 1) (layer B.Cu) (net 22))
 (segment (start 109.725 98.925) (end 113 102.2) (width 1) (layer B.Cu) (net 22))
 (segment (start 113 102.2) (end 113 112.3) (width 1) (layer B.Cu) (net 22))
 (segment (start 106.175 101.465) (end 107.765 101.465) (width 1) (layer B.Cu) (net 24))
 (segment (start 107.765 101.465) (end 110.35 104.05) (width 1) (layer B.Cu) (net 24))
 (segment (start 110.35 104.05) (end 110.35 113.15) (width 1) (layer B.Cu) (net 24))
 (segment (start 110.35 113.15) (end 112.04 114.84) (width 1) (layer B.Cu) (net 24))
 (segment (start 112.04 114.84) (end 113 114.84) (width 1) (layer B.Cu) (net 24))
 (segment (start 106.175 104.005) (end 106.955 104.005) (width 1) (layer B.Cu) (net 26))
 (segment (start 106.955 104.005) (end 108.8 105.85) (width 1) (layer B.Cu) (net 26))
 (segment (start 108.8 105.85) (end 108.8 115.85) (width 1) (layer B.Cu) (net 26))
 (segment (start 108.8 115.85) (end 110.33 117.38) (width 1) (layer B.Cu) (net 26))
 (segment (start 110.33 117.38) (end 113 117.38) (width 1) (layer B.Cu) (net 26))
 (segment (start 106.175 121.785) (end 108.015 121.785) (width 1) (layer B.Cu) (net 40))
 (segment (start 108.015 121.785) (end 109.88 119.92) (width 1) (layer B.Cu) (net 40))
 (segment (start 109.88 119.92) (end 113 119.92) (width 1) (layer B.Cu) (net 40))
 (segment (start 106.175 124.325) (end 108.325 124.325) (width 1) (layer B.Cu) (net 42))
 (segment (start 108.325 124.325) (end 110.19 122.46) (width 1) (layer B.Cu) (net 42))
 (segment (start 110.19 122.46) (end 113 122.46) (width 1) (layer B.Cu) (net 42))
 (segment (start 106.175 126.865) (end 108.485 126.865) (width 1) (layer B.Cu) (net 44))
 (segment (start 108.485 126.865) (end 110.35 125) (width 1) (layer B.Cu) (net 44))
 (segment (start 110.35 125) (end 113 125) (width 1) (layer B.Cu) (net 44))
 (segment (start 106.255 131.865) (end 106.175 131.945) (width 1) (layer B.Cu) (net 48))
 (segment (start 106.175 131.945) (end 107.305 131.945) (width 1) (layer B.Cu) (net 48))
 (segment (start 107.305 131.945) (end 111.71 127.54) (width 1) (layer B.Cu) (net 48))
 (segment (start 111.71 127.54) (end 113 127.54) (width 1) (layer B.Cu) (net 48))
 (segment (start 120.62 117.38) (end 126.37 117.38) (width 1) (layer B.Cu) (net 56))
 (segment (start 126.37 117.38) (end 128.775 114.975) (width 1) (layer B.Cu) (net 56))
 (segment (start 128.775 114.975) (end 128.775 112.975) (width 1) (layer B.Cu) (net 56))
 (segment (start 120.62 125) (end 144.75 125) (width 1) (layer B.Cu) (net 53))
 (segment (start 144.75 125) (end 146.775 122.975) (width 1) (layer B.Cu) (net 53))
 (segment (start 122.8 108.4) (end 122.8 110) (width 1) (layer B.Cu) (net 57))
 (segment (start 122.8 110) (end 123.25 110.45) (width 1) (layer B.Cu) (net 57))
 (segment (start 123.25 110.45) (end 123.25 113.7) (width 1) (layer B.Cu) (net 57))
 (segment (start 123.25 113.7) (end 122.11 114.84) (width 1) (layer B.Cu) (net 57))
 (segment (start 122.11 114.84) (end 120.62 114.84) (width 1) (layer B.Cu) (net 57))
 (segment (start 120.62 122.46) (end 138.29 122.46) (width 1) (layer B.Cu) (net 54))
 (segment (start 138.29 122.46) (end 140.775 119.975) (width 1) (layer B.Cu) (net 54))
 (segment (start 116.775 104.975) (end 116.775 107.025) (width 1) (layer B.Cu) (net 58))
 (segment (start 116.775 107.025) (end 120.62 110.87) (width 1) (layer B.Cu) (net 58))
 (segment (start 120.62 110.87) (end 120.62 112.3) (width 1) (layer B.Cu) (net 58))
 (segment (start 120.62 119.92) (end 132.63 119.92) (width 1) (layer B.Cu) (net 55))
 (segment (start 132.63 119.92) (end 134.775 117.775) (width 1) (layer B.Cu) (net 55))
 (segment (start 134.775 117.775) (end 134.775 115.975) (width 1) (layer B.Cu) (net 55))
 (segment (start 120.62 127.54) (end 151.21 127.54) (width 1) (layer B.Cu) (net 52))
 (segment (start 151.21 127.54) (end 152.775 125.975) (width 1) (layer B.Cu) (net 52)))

